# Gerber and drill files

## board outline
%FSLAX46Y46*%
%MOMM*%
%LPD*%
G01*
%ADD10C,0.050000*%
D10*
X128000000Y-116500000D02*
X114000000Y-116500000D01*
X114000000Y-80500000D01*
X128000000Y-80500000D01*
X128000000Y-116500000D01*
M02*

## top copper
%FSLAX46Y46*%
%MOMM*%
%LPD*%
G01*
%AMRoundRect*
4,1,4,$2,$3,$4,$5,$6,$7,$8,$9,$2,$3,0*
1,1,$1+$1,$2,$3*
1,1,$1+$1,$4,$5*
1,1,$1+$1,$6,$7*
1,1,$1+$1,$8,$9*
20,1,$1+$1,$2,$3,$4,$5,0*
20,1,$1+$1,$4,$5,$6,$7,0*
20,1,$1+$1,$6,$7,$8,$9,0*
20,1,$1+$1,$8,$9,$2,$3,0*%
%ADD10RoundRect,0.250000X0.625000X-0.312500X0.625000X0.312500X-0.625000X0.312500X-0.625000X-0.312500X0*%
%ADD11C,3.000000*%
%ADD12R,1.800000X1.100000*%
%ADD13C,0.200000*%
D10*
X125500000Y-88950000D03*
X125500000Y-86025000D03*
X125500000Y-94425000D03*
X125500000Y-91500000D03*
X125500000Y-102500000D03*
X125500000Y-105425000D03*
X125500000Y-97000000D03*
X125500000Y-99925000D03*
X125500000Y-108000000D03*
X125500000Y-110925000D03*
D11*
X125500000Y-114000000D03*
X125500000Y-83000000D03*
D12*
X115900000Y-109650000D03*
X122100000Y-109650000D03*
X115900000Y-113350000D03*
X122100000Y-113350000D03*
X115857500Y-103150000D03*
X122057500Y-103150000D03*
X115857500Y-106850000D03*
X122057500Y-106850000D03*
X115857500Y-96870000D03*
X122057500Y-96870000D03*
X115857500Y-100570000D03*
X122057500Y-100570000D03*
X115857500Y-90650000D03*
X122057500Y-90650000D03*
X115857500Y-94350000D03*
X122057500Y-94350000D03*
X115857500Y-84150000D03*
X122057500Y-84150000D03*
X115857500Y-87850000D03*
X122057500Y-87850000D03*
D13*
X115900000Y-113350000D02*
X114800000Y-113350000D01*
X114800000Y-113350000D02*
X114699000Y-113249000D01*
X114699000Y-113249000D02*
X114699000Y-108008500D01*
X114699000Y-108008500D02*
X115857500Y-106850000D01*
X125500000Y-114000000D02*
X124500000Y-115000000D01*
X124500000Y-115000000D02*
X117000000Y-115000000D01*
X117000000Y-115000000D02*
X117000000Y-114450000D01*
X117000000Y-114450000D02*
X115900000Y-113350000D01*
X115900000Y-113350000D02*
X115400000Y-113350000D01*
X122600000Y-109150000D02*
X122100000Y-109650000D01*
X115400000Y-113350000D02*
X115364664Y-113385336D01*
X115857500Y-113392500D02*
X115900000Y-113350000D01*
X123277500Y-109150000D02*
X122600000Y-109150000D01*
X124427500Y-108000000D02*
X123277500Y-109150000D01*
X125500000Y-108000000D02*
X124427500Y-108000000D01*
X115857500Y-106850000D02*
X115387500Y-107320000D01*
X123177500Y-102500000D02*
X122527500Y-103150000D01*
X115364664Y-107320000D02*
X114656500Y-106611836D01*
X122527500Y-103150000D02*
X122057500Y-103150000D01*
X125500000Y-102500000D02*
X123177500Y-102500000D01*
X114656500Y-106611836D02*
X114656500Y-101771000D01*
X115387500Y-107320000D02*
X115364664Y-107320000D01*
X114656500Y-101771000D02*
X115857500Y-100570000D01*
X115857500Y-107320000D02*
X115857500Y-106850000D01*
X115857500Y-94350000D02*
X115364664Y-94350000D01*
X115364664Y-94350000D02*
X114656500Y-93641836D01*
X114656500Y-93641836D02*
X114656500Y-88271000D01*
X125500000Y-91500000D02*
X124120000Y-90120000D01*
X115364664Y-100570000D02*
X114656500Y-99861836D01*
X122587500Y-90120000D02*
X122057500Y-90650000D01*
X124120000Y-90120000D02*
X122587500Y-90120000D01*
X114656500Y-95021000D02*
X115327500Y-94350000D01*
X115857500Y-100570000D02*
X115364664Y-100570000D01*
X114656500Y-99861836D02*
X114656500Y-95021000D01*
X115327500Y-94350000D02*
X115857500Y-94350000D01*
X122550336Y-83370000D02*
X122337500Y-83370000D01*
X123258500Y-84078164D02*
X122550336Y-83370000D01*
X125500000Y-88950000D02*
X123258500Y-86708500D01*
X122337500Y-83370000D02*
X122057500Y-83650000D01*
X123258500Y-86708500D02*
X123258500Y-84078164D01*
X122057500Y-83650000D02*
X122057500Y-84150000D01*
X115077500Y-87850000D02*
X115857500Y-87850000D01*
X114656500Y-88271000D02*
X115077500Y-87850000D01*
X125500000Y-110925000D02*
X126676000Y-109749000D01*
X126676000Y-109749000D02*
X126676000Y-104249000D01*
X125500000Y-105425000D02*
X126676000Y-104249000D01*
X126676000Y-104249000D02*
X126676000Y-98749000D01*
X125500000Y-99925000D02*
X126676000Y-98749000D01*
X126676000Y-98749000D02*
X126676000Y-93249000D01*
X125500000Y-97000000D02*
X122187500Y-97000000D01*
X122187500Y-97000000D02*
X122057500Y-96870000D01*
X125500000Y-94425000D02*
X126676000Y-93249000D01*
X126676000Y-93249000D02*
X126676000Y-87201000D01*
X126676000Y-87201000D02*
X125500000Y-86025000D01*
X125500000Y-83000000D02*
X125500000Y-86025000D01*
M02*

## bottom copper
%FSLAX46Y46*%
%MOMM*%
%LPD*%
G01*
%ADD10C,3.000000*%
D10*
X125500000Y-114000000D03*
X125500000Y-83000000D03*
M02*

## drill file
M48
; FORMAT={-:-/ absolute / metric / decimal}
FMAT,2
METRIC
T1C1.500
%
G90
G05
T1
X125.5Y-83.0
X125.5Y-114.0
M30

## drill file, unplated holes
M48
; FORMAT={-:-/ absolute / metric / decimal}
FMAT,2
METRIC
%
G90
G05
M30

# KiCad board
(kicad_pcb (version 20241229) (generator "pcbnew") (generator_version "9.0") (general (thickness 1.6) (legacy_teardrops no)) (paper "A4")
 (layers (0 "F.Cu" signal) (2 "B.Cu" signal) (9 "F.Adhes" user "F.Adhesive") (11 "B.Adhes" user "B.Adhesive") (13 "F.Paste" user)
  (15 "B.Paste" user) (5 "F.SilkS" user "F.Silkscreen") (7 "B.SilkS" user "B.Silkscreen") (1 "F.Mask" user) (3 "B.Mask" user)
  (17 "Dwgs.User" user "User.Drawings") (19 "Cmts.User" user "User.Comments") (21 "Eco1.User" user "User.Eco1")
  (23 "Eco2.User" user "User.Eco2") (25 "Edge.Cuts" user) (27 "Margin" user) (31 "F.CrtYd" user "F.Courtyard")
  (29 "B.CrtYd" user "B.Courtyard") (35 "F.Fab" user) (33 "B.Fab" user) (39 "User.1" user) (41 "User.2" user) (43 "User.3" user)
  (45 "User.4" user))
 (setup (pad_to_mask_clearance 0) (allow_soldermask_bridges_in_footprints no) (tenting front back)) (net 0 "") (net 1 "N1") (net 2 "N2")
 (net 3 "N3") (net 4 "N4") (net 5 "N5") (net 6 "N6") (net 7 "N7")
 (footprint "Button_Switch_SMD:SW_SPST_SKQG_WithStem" (layer "F.Cu") (at 118.9575 86)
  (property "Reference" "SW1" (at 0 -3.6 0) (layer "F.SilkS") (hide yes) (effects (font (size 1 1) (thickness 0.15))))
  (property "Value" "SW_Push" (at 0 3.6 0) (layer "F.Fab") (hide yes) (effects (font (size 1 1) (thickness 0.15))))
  (pad "1" smd rect (at -3.1 -1.85) (size 1.8 1.1) (layers "F.Cu" "F.Mask" "F.Paste") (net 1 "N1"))
  (pad "1" smd rect (at 3.1 -1.85) (size 1.8 1.1) (layers "F.Cu" "F.Mask" "F.Paste") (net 1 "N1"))
  (pad "2" smd rect (at -3.1 1.85) (size 1.8 1.1) (layers "F.Cu" "F.Mask" "F.Paste") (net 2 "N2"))
  (pad "2" smd rect (at 3.1 1.85) (size 1.8 1.1) (layers "F.Cu" "F.Mask" "F.Paste") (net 2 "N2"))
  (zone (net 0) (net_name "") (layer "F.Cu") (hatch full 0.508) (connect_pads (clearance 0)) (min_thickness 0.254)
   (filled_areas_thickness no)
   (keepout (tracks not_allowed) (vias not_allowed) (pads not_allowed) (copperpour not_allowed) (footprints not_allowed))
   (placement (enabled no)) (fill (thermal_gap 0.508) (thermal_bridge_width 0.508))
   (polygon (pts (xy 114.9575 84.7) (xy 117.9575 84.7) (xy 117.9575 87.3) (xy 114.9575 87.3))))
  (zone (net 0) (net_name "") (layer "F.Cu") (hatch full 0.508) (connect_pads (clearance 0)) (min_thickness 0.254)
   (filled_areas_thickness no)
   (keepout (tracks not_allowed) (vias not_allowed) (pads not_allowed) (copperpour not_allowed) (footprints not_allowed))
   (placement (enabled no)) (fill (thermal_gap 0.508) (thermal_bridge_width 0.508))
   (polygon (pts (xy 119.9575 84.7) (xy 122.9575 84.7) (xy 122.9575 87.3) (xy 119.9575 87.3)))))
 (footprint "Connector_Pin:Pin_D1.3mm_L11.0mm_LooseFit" (layer "F.Cu") (at 125.5 114)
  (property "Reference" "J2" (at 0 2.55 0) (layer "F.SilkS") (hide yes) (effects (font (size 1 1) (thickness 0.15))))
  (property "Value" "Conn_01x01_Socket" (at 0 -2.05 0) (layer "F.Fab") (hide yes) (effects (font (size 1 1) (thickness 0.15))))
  (pad "1" thru_hole circle (at 0 0) (size 3 3) (drill 1.5) (layers "*.Cu" "*.Mask") (remove_unused_layers no) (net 2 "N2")))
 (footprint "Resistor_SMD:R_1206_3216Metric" (layer "F.Cu") (at 125.5 98.4625 90)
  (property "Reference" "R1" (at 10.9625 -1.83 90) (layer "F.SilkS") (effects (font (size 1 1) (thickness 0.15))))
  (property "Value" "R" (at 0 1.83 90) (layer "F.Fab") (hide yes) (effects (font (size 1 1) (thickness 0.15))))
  (pad "1" smd roundrect (at -1.4625 0 90) (size 1.125 1.75) (layers "F.Cu" "F.Mask" "F.Paste") (roundrect_rratio 0.222222) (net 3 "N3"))
  (pad "2" smd roundrect (at 1.4625 0 90) (size 1.125 1.75) (layers "F.Cu" "F.Mask" "F.Paste") (roundrect_rratio 0.222222) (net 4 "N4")))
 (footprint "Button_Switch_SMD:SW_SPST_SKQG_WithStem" (layer "F.Cu") (at 118.9575 98.72)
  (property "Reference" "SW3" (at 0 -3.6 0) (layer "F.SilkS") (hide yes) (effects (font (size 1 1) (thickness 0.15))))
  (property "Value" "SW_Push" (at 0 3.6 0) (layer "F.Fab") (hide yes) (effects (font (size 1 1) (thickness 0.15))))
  (pad "1" smd rect (at -3.1 -1.85) (size 1.8 1.1) (layers "F.Cu" "F.Mask" "F.Paste") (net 4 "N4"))
  (pad "1" smd rect (at 3.1 -1.85) (size 1.8 1.1) (layers "F.Cu" "F.Mask" "F.Paste") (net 4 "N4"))
  (pad "2" smd rect (at -3.1 1.85) (size 1.8 1.1) (layers "F.Cu" "F.Mask" "F.Paste") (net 2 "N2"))
  (pad "2" smd rect (at 3.1 1.85) (size 1.8 1.1) (layers "F.Cu" "F.Mask" "F.Paste") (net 2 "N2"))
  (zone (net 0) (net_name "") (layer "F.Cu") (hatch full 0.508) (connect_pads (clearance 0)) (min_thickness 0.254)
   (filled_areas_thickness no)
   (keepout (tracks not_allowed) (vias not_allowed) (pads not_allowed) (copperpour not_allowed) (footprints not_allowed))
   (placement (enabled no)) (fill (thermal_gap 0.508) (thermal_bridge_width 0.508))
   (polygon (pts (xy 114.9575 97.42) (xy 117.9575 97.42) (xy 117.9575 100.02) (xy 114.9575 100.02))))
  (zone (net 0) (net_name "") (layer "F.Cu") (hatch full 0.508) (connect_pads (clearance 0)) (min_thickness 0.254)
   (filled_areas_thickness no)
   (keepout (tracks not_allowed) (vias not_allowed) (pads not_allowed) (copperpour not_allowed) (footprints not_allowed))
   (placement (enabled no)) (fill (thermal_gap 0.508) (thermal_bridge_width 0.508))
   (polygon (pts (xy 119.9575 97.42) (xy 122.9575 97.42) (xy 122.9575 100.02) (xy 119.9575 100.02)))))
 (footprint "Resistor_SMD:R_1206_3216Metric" (layer "F.Cu") (at 125.5 92.9625 90)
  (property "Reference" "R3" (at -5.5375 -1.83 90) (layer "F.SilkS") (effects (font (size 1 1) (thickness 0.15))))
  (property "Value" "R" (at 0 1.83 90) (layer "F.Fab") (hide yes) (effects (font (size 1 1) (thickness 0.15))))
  (pad "1" smd roundrect (at -1.4625 0 90) (size 1.125 1.75) (layers "F.Cu" "F.Mask" "F.Paste") (roundrect_rratio 0.222222) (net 3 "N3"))
  (pad "2" smd roundrect (at 1.4625 0 90) (size 1.125 1.75) (layers "F.Cu" "F.Mask" "F.Paste") (roundrect_rratio 0.222222) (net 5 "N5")))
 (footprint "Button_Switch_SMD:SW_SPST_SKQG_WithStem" (layer "F.Cu") (at 118.9575 92.5)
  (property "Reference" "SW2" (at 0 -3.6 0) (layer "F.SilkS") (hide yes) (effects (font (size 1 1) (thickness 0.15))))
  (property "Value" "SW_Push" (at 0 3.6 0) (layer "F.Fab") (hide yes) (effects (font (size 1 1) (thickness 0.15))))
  (pad "1" smd rect (at -3.1 -1.85) (size 1.8 1.1) (layers "F.Cu" "F.Mask" "F.Paste") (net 5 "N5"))
  (pad "1" smd rect (at 3.1 -1.85) (size 1.8 1.1) (layers "F.Cu" "F.Mask" "F.Paste") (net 5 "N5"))
  (pad "2" smd rect (at -3.1 1.85) (size 1.8 1.1) (layers "F.Cu" "F.Mask" "F.Paste") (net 2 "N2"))
  (pad "2" smd rect (at 3.1 1.85) (size 1.8 1.1) (layers "F.Cu" "F.Mask" "F.Paste") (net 2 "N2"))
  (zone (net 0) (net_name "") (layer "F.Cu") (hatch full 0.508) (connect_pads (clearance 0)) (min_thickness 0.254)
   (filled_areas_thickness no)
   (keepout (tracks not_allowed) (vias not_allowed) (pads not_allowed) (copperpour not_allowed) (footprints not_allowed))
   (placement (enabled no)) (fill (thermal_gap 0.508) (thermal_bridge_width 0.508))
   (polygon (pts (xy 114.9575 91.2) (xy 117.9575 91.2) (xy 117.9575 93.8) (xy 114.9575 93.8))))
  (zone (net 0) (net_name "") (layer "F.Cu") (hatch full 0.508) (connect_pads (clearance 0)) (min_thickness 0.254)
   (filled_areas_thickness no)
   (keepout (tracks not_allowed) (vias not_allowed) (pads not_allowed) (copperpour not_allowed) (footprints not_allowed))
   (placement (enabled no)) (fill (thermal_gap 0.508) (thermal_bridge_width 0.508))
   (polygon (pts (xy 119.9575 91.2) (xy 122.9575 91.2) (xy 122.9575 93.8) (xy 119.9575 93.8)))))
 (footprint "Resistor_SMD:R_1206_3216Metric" (layer "F.Cu") (at 125.5 109.4625 90)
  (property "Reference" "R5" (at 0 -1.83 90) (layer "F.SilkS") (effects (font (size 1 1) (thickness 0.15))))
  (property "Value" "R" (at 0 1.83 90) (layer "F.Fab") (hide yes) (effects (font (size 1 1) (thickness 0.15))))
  (pad "1" smd roundrect (at -1.4625 0 90) (size 1.125 1.75) (layers "F.Cu" "F.Mask" "F.Paste") (roundrect_rratio 0.222222) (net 3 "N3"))
  (pad "2" smd roundrect (at 1.4625 0 90) (size 1.125 1.75) (layers "F.Cu" "F.Mask" "F.Paste") (roundrect_rratio 0.222222) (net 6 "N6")))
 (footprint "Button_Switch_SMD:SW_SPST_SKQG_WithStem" (layer "F.Cu") (at 118.9575 105)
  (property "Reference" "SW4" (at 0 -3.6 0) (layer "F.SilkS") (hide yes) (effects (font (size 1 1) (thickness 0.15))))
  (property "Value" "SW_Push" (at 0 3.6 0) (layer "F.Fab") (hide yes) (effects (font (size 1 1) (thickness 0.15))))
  (pad "1" smd rect (at -3.1 -1.85) (size 1.8 1.1) (layers "F.Cu" "F.Mask" "F.Paste") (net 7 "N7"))
  (pad "1" smd rect (at 3.1 -1.85) (size 1.8 1.1) (layers "F.Cu" "F.Mask" "F.Paste") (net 7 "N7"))
  (pad "2" smd rect (at -3.1 1.85) (size 1.8 1.1) (layers "F.Cu" "F.Mask" "F.Paste") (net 2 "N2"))
  (pad "2" smd rect (at 3.1 1.85) (size 1.8 1.1) (layers "F.Cu" "F.Mask" "F.Paste") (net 2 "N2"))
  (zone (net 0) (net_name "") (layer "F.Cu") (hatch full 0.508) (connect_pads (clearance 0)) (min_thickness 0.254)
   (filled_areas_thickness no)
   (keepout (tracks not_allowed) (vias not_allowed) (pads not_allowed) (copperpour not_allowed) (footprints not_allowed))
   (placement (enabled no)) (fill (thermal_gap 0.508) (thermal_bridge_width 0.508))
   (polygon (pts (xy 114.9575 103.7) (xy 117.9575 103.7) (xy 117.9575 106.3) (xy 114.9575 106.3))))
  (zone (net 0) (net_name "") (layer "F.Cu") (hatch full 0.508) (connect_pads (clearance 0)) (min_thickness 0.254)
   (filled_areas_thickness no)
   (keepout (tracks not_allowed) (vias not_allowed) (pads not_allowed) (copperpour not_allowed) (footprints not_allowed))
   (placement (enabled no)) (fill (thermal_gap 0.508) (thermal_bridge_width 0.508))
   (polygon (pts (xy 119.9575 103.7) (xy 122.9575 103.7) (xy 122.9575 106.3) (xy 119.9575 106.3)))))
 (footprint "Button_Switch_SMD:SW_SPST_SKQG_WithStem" (layer "F.Cu") (at 119 111.5)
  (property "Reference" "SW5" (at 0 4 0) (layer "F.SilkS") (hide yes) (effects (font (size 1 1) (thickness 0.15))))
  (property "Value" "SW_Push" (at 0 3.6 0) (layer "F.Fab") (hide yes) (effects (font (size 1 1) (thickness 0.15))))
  (pad "1" smd rect (at -3.1 -1.85) (size 1.8 1.1) (layers "F.Cu" "F.Mask" "F.Paste") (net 6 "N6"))
  (pad "1" smd rect (at 3.1 -1.85) (size 1.8 1.1) (layers "F.Cu" "F.Mask" "F.Paste") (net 6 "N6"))
  (pad "2" smd rect (at -3.1 1.85) (size 1.8 1.1) (layers "F.Cu" "F.Mask" "F.Paste") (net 2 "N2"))
  (pad "2" smd rect (at 3.1 1.85) (size 1.8 1.1) (layers "F.Cu" "F.Mask" "F.Paste") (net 2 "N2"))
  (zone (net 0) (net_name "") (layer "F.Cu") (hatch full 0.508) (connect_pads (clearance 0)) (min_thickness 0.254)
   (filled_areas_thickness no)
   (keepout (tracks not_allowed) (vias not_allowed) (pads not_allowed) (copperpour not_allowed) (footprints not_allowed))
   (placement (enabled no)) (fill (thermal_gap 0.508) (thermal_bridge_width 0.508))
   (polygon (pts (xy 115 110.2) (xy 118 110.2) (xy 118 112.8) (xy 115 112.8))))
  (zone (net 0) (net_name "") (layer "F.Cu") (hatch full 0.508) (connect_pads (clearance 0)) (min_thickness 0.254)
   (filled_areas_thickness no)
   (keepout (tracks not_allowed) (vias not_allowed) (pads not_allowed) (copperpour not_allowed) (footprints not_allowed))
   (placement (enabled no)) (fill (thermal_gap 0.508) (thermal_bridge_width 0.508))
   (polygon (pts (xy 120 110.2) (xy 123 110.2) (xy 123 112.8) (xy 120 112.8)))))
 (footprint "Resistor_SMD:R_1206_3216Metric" (layer "F.Cu") (at 125.5 103.9625 90)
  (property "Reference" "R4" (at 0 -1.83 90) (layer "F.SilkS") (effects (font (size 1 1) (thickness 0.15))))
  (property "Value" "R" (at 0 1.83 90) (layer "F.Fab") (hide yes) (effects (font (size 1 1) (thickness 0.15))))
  (pad "1" smd roundrect (at -1.4625 0 90) (size 1.125 1.75) (layers "F.Cu" "F.Mask" "F.Paste") (roundrect_rratio 0.222222) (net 3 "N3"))
  (pad "2" smd roundrect (at 1.4625 0 90) (size 1.125 1.75) (layers "F.Cu" "F.Mask" "F.Paste") (roundrect_rratio 0.222222) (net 7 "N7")))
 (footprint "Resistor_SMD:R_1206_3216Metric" (layer "F.Cu") (at 125.5 87.4875 90)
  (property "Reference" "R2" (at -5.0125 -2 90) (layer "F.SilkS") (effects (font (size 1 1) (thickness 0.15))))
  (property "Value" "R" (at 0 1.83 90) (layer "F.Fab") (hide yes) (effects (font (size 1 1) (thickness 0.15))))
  (pad "1" smd roundrect (at -1.4625 0 90) (size 1.125 1.75) (layers "F.Cu" "F.Mask" "F.Paste") (roundrect_rratio 0.222222) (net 1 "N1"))
  (pad "2" smd roundrect (at 1.4625 0 90) (size 1.125 1.75) (layers "F.Cu" "F.Mask" "F.Paste") (roundrect_rratio 0.222222) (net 3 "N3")))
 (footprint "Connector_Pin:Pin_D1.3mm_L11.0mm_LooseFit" (layer "F.Cu") (at 125.5 83 180)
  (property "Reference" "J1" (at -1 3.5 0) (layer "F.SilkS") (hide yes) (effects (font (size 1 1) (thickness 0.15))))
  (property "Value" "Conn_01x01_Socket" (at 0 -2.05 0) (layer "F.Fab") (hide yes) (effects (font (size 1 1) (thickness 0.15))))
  (pad "1" thru_hole circle (at 0 0 180) (size 3 3) (drill 1.5) (layers "*.Cu" "*.Mask") (remove_unused_layers no) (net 3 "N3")))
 (gr_poly (pts (xy 114 80.5) (xy 128 80.5) (xy 128 116.5) (xy 114 116.5)) (stroke (width 0.05) (type solid)) (fill no) (layer "Edge.Cuts"))
 (segment (start 125.5 99.925) (end 126.676 98.749) (width 0.2) (layer "F.Cu") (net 3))
 (segment (start 125.5 110.925) (end 126.676 109.749) (width 0.2) (layer "F.Cu") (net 3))
 (segment (start 126.676 98.749) (end 126.676 93.249) (width 0.2) (layer "F.Cu") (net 3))
 (segment (start 125.5 83) (end 125.5 86.025) (width 0.2) (layer "F.Cu") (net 3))
 (segment (start 126.676 104.249) (end 126.676 98.749) (width 0.2) (layer "F.Cu") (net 3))
 (segment (start 125.5 105.425) (end 126.676 104.249) (width 0.2) (layer "F.Cu") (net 3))
 (segment (start 126.676 87.201) (end 125.5 86.025) (width 0.2) (layer "F.Cu") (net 3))
 (segment (start 126.676 93.249) (end 126.676 87.201) (width 0.2) (layer "F.Cu") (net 3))
 (segment (start 126.676 109.749) (end 126.676 104.249) (width 0.2) (layer "F.Cu") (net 3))
 (segment (start 125.5 94.425) (end 126.676 93.249) (width 0.2) (layer "F.Cu") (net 3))
 (segment (start 114.6565 93.641836) (end 114.6565 88.271) (width 0.2) (layer "F.Cu") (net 2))
 (segment (start 115.3875 107.32) (end 115.364664 107.32) (width 0.2) (layer "F.Cu") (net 2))
 (segment (start 114.6565 95.021) (end 115.3275 94.35) (width 0.2) (layer "F.Cu") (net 2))
 (segment (start 115.364664 100.57) (end 114.6565 99.861836) (width 0.2) (layer "F.Cu") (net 2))
 (segment (start 114.8 113.35) (end 114.699 113.249) (width 0.2) (layer "F.Cu") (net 2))
 (segment (start 117 115) (end 117 114.45) (width 0.2) (layer "F.Cu") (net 2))
 (segment (start 115.8575 113.3925) (end 115.9 113.35) (width 0.2) (layer "F.Cu") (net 2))
 (segment (start 115.0775 87.85) (end 115.8575 87.85) (width 0.2) (layer "F.Cu") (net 2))
 (segment (start 114.6565 88.271) (end 115.0775 87.85) (width 0.2) (layer "F.Cu") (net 2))
 (segment (start 115.4 113.35) (end 115.364664 113.385336) (width 0.2) (layer "F.Cu") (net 2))
 (segment (start 117 114.45) (end 115.9 113.35) (width 0.2) (layer "F.Cu") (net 2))
 (segment (start 115.3275 94.35) (end 115.8575 94.35) (width 0.2) (layer "F.Cu") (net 2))
 (segment (start 114.6565 101.771) (end 115.8575 100.57) (width 0.2) (layer "F.Cu") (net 2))
 (segment (start 125.5 114) (end 124.5 115) (width 0.2) (layer "F.Cu") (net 2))
 (segment (start 115.364664 107.32) (end 114.6565 106.611836) (width 0.2) (layer "F.Cu") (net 2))
 (segment (start 114.6565 106.611836) (end 114.6565 101.771) (width 0.2) (layer "F.Cu") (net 2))
 (segment (start 115.8575 106.85) (end 115.3875 107.32) (width 0.2) (layer "F.Cu") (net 2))
 (segment (start 115.8575 100.57) (end 115.364664 100.57) (width 0.2) (layer "F.Cu") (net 2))
 (segment (start 115.9 113.35) (end 115.4 113.35) (width 0.2) (layer "F.Cu") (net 2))
 (segment (start 114.699 108.0085) (end 115.8575 106.85) (width 0.2) (layer "F.Cu") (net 2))
 (segment (start 115.9 113.35) (end 114.8 113.35) (width 0.2) (layer "F.Cu") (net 2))
 (segment (start 124.5 115) (end 117 115) (width 0.2) (layer "F.Cu") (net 2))
 (segment (start 115.364664 94.35) (end 114.6565 93.641836) (width 0.2) (layer "F.Cu") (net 2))
 (segment (start 114.6565 99.861836) (end 114.6565 95.021) (width 0.2) (layer "F.Cu") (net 2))
 (segment (start 115.8575 94.35) (end 115.364664 94.35) (width 0.2) (layer "F.Cu") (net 2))
 (segment (start 115.8575 107.32) (end 115.8575 106.85) (width 0.2) (layer "F.Cu") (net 2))
 (segment (start 114.699 113.249) (end 114.699 108.0085) (width 0.2) (layer "F.Cu") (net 2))
 (segment (start 122.1875 97) (end 122.0575 96.87) (width 0.2) (layer "F.Cu") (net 4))
 (segment (start 125.5 97) (end 122.1875 97) (width 0.2) (layer "F.Cu") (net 4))
 (segment (start 123.2585 84.078164) (end 122.550336 83.37) (width 0.2) (layer "F.Cu") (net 1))
 (segment (start 122.3375 83.37) (end 122.0575 83.65) (width 0.2) (layer "F.Cu") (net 1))
 (segment (start 122.550336 83.37) (end 122.3375 83.37) (width 0.2) (layer "F.Cu") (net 1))
 (segment (start 125.5 88.95) (end 123.2585 86.7085) (width 0.2) (layer "F.Cu") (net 1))
 (segment (start 122.0575 83.65) (end 122.0575 84.15) (width 0.2) (layer "F.Cu") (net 1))
 (segment (start 123.2585 86.7085) (end 123.2585 84.078164) (width 0.2) (layer "F.Cu") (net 1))
 (segment (start 125.5 91.5) (end 124.12 90.12) (width 0.2) (layer "F.Cu") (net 5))
 (segment (start 122.5875 90.12) (end 122.0575 90.65) (width 0.2) (layer "F.Cu") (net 5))
 (segment (start 124.12 90.12) (end 122.5875 90.12) (width 0.2) (layer "F.Cu") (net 5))
 (segment (start 125.5 102.5) (end 123.1775 102.5) (width 0.2) (layer "F.Cu") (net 7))
 (segment (start 123.1775 102.5) (end 122.5275 103.15) (width 0.2) (layer "F.Cu") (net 7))
 (segment (start 122.5275 103.15) (end 122.0575 103.15) (width 0.2) (layer "F.Cu") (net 7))
 (segment (start 122.6 109.15) (end 122.1 109.65) (width 0.2) (layer "F.Cu") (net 6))
 (segment (start 123.2775 109.15) (end 122.6 109.15) (width 0.2) (layer "F.Cu") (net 6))
 (segment (start 125.5 108) (end 124.4275 108) (width 0.2) (layer "F.Cu") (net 6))
 (segment (start 124.4275 108) (end 123.2775 109.15) (width 0.2) (layer "F.Cu") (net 6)))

